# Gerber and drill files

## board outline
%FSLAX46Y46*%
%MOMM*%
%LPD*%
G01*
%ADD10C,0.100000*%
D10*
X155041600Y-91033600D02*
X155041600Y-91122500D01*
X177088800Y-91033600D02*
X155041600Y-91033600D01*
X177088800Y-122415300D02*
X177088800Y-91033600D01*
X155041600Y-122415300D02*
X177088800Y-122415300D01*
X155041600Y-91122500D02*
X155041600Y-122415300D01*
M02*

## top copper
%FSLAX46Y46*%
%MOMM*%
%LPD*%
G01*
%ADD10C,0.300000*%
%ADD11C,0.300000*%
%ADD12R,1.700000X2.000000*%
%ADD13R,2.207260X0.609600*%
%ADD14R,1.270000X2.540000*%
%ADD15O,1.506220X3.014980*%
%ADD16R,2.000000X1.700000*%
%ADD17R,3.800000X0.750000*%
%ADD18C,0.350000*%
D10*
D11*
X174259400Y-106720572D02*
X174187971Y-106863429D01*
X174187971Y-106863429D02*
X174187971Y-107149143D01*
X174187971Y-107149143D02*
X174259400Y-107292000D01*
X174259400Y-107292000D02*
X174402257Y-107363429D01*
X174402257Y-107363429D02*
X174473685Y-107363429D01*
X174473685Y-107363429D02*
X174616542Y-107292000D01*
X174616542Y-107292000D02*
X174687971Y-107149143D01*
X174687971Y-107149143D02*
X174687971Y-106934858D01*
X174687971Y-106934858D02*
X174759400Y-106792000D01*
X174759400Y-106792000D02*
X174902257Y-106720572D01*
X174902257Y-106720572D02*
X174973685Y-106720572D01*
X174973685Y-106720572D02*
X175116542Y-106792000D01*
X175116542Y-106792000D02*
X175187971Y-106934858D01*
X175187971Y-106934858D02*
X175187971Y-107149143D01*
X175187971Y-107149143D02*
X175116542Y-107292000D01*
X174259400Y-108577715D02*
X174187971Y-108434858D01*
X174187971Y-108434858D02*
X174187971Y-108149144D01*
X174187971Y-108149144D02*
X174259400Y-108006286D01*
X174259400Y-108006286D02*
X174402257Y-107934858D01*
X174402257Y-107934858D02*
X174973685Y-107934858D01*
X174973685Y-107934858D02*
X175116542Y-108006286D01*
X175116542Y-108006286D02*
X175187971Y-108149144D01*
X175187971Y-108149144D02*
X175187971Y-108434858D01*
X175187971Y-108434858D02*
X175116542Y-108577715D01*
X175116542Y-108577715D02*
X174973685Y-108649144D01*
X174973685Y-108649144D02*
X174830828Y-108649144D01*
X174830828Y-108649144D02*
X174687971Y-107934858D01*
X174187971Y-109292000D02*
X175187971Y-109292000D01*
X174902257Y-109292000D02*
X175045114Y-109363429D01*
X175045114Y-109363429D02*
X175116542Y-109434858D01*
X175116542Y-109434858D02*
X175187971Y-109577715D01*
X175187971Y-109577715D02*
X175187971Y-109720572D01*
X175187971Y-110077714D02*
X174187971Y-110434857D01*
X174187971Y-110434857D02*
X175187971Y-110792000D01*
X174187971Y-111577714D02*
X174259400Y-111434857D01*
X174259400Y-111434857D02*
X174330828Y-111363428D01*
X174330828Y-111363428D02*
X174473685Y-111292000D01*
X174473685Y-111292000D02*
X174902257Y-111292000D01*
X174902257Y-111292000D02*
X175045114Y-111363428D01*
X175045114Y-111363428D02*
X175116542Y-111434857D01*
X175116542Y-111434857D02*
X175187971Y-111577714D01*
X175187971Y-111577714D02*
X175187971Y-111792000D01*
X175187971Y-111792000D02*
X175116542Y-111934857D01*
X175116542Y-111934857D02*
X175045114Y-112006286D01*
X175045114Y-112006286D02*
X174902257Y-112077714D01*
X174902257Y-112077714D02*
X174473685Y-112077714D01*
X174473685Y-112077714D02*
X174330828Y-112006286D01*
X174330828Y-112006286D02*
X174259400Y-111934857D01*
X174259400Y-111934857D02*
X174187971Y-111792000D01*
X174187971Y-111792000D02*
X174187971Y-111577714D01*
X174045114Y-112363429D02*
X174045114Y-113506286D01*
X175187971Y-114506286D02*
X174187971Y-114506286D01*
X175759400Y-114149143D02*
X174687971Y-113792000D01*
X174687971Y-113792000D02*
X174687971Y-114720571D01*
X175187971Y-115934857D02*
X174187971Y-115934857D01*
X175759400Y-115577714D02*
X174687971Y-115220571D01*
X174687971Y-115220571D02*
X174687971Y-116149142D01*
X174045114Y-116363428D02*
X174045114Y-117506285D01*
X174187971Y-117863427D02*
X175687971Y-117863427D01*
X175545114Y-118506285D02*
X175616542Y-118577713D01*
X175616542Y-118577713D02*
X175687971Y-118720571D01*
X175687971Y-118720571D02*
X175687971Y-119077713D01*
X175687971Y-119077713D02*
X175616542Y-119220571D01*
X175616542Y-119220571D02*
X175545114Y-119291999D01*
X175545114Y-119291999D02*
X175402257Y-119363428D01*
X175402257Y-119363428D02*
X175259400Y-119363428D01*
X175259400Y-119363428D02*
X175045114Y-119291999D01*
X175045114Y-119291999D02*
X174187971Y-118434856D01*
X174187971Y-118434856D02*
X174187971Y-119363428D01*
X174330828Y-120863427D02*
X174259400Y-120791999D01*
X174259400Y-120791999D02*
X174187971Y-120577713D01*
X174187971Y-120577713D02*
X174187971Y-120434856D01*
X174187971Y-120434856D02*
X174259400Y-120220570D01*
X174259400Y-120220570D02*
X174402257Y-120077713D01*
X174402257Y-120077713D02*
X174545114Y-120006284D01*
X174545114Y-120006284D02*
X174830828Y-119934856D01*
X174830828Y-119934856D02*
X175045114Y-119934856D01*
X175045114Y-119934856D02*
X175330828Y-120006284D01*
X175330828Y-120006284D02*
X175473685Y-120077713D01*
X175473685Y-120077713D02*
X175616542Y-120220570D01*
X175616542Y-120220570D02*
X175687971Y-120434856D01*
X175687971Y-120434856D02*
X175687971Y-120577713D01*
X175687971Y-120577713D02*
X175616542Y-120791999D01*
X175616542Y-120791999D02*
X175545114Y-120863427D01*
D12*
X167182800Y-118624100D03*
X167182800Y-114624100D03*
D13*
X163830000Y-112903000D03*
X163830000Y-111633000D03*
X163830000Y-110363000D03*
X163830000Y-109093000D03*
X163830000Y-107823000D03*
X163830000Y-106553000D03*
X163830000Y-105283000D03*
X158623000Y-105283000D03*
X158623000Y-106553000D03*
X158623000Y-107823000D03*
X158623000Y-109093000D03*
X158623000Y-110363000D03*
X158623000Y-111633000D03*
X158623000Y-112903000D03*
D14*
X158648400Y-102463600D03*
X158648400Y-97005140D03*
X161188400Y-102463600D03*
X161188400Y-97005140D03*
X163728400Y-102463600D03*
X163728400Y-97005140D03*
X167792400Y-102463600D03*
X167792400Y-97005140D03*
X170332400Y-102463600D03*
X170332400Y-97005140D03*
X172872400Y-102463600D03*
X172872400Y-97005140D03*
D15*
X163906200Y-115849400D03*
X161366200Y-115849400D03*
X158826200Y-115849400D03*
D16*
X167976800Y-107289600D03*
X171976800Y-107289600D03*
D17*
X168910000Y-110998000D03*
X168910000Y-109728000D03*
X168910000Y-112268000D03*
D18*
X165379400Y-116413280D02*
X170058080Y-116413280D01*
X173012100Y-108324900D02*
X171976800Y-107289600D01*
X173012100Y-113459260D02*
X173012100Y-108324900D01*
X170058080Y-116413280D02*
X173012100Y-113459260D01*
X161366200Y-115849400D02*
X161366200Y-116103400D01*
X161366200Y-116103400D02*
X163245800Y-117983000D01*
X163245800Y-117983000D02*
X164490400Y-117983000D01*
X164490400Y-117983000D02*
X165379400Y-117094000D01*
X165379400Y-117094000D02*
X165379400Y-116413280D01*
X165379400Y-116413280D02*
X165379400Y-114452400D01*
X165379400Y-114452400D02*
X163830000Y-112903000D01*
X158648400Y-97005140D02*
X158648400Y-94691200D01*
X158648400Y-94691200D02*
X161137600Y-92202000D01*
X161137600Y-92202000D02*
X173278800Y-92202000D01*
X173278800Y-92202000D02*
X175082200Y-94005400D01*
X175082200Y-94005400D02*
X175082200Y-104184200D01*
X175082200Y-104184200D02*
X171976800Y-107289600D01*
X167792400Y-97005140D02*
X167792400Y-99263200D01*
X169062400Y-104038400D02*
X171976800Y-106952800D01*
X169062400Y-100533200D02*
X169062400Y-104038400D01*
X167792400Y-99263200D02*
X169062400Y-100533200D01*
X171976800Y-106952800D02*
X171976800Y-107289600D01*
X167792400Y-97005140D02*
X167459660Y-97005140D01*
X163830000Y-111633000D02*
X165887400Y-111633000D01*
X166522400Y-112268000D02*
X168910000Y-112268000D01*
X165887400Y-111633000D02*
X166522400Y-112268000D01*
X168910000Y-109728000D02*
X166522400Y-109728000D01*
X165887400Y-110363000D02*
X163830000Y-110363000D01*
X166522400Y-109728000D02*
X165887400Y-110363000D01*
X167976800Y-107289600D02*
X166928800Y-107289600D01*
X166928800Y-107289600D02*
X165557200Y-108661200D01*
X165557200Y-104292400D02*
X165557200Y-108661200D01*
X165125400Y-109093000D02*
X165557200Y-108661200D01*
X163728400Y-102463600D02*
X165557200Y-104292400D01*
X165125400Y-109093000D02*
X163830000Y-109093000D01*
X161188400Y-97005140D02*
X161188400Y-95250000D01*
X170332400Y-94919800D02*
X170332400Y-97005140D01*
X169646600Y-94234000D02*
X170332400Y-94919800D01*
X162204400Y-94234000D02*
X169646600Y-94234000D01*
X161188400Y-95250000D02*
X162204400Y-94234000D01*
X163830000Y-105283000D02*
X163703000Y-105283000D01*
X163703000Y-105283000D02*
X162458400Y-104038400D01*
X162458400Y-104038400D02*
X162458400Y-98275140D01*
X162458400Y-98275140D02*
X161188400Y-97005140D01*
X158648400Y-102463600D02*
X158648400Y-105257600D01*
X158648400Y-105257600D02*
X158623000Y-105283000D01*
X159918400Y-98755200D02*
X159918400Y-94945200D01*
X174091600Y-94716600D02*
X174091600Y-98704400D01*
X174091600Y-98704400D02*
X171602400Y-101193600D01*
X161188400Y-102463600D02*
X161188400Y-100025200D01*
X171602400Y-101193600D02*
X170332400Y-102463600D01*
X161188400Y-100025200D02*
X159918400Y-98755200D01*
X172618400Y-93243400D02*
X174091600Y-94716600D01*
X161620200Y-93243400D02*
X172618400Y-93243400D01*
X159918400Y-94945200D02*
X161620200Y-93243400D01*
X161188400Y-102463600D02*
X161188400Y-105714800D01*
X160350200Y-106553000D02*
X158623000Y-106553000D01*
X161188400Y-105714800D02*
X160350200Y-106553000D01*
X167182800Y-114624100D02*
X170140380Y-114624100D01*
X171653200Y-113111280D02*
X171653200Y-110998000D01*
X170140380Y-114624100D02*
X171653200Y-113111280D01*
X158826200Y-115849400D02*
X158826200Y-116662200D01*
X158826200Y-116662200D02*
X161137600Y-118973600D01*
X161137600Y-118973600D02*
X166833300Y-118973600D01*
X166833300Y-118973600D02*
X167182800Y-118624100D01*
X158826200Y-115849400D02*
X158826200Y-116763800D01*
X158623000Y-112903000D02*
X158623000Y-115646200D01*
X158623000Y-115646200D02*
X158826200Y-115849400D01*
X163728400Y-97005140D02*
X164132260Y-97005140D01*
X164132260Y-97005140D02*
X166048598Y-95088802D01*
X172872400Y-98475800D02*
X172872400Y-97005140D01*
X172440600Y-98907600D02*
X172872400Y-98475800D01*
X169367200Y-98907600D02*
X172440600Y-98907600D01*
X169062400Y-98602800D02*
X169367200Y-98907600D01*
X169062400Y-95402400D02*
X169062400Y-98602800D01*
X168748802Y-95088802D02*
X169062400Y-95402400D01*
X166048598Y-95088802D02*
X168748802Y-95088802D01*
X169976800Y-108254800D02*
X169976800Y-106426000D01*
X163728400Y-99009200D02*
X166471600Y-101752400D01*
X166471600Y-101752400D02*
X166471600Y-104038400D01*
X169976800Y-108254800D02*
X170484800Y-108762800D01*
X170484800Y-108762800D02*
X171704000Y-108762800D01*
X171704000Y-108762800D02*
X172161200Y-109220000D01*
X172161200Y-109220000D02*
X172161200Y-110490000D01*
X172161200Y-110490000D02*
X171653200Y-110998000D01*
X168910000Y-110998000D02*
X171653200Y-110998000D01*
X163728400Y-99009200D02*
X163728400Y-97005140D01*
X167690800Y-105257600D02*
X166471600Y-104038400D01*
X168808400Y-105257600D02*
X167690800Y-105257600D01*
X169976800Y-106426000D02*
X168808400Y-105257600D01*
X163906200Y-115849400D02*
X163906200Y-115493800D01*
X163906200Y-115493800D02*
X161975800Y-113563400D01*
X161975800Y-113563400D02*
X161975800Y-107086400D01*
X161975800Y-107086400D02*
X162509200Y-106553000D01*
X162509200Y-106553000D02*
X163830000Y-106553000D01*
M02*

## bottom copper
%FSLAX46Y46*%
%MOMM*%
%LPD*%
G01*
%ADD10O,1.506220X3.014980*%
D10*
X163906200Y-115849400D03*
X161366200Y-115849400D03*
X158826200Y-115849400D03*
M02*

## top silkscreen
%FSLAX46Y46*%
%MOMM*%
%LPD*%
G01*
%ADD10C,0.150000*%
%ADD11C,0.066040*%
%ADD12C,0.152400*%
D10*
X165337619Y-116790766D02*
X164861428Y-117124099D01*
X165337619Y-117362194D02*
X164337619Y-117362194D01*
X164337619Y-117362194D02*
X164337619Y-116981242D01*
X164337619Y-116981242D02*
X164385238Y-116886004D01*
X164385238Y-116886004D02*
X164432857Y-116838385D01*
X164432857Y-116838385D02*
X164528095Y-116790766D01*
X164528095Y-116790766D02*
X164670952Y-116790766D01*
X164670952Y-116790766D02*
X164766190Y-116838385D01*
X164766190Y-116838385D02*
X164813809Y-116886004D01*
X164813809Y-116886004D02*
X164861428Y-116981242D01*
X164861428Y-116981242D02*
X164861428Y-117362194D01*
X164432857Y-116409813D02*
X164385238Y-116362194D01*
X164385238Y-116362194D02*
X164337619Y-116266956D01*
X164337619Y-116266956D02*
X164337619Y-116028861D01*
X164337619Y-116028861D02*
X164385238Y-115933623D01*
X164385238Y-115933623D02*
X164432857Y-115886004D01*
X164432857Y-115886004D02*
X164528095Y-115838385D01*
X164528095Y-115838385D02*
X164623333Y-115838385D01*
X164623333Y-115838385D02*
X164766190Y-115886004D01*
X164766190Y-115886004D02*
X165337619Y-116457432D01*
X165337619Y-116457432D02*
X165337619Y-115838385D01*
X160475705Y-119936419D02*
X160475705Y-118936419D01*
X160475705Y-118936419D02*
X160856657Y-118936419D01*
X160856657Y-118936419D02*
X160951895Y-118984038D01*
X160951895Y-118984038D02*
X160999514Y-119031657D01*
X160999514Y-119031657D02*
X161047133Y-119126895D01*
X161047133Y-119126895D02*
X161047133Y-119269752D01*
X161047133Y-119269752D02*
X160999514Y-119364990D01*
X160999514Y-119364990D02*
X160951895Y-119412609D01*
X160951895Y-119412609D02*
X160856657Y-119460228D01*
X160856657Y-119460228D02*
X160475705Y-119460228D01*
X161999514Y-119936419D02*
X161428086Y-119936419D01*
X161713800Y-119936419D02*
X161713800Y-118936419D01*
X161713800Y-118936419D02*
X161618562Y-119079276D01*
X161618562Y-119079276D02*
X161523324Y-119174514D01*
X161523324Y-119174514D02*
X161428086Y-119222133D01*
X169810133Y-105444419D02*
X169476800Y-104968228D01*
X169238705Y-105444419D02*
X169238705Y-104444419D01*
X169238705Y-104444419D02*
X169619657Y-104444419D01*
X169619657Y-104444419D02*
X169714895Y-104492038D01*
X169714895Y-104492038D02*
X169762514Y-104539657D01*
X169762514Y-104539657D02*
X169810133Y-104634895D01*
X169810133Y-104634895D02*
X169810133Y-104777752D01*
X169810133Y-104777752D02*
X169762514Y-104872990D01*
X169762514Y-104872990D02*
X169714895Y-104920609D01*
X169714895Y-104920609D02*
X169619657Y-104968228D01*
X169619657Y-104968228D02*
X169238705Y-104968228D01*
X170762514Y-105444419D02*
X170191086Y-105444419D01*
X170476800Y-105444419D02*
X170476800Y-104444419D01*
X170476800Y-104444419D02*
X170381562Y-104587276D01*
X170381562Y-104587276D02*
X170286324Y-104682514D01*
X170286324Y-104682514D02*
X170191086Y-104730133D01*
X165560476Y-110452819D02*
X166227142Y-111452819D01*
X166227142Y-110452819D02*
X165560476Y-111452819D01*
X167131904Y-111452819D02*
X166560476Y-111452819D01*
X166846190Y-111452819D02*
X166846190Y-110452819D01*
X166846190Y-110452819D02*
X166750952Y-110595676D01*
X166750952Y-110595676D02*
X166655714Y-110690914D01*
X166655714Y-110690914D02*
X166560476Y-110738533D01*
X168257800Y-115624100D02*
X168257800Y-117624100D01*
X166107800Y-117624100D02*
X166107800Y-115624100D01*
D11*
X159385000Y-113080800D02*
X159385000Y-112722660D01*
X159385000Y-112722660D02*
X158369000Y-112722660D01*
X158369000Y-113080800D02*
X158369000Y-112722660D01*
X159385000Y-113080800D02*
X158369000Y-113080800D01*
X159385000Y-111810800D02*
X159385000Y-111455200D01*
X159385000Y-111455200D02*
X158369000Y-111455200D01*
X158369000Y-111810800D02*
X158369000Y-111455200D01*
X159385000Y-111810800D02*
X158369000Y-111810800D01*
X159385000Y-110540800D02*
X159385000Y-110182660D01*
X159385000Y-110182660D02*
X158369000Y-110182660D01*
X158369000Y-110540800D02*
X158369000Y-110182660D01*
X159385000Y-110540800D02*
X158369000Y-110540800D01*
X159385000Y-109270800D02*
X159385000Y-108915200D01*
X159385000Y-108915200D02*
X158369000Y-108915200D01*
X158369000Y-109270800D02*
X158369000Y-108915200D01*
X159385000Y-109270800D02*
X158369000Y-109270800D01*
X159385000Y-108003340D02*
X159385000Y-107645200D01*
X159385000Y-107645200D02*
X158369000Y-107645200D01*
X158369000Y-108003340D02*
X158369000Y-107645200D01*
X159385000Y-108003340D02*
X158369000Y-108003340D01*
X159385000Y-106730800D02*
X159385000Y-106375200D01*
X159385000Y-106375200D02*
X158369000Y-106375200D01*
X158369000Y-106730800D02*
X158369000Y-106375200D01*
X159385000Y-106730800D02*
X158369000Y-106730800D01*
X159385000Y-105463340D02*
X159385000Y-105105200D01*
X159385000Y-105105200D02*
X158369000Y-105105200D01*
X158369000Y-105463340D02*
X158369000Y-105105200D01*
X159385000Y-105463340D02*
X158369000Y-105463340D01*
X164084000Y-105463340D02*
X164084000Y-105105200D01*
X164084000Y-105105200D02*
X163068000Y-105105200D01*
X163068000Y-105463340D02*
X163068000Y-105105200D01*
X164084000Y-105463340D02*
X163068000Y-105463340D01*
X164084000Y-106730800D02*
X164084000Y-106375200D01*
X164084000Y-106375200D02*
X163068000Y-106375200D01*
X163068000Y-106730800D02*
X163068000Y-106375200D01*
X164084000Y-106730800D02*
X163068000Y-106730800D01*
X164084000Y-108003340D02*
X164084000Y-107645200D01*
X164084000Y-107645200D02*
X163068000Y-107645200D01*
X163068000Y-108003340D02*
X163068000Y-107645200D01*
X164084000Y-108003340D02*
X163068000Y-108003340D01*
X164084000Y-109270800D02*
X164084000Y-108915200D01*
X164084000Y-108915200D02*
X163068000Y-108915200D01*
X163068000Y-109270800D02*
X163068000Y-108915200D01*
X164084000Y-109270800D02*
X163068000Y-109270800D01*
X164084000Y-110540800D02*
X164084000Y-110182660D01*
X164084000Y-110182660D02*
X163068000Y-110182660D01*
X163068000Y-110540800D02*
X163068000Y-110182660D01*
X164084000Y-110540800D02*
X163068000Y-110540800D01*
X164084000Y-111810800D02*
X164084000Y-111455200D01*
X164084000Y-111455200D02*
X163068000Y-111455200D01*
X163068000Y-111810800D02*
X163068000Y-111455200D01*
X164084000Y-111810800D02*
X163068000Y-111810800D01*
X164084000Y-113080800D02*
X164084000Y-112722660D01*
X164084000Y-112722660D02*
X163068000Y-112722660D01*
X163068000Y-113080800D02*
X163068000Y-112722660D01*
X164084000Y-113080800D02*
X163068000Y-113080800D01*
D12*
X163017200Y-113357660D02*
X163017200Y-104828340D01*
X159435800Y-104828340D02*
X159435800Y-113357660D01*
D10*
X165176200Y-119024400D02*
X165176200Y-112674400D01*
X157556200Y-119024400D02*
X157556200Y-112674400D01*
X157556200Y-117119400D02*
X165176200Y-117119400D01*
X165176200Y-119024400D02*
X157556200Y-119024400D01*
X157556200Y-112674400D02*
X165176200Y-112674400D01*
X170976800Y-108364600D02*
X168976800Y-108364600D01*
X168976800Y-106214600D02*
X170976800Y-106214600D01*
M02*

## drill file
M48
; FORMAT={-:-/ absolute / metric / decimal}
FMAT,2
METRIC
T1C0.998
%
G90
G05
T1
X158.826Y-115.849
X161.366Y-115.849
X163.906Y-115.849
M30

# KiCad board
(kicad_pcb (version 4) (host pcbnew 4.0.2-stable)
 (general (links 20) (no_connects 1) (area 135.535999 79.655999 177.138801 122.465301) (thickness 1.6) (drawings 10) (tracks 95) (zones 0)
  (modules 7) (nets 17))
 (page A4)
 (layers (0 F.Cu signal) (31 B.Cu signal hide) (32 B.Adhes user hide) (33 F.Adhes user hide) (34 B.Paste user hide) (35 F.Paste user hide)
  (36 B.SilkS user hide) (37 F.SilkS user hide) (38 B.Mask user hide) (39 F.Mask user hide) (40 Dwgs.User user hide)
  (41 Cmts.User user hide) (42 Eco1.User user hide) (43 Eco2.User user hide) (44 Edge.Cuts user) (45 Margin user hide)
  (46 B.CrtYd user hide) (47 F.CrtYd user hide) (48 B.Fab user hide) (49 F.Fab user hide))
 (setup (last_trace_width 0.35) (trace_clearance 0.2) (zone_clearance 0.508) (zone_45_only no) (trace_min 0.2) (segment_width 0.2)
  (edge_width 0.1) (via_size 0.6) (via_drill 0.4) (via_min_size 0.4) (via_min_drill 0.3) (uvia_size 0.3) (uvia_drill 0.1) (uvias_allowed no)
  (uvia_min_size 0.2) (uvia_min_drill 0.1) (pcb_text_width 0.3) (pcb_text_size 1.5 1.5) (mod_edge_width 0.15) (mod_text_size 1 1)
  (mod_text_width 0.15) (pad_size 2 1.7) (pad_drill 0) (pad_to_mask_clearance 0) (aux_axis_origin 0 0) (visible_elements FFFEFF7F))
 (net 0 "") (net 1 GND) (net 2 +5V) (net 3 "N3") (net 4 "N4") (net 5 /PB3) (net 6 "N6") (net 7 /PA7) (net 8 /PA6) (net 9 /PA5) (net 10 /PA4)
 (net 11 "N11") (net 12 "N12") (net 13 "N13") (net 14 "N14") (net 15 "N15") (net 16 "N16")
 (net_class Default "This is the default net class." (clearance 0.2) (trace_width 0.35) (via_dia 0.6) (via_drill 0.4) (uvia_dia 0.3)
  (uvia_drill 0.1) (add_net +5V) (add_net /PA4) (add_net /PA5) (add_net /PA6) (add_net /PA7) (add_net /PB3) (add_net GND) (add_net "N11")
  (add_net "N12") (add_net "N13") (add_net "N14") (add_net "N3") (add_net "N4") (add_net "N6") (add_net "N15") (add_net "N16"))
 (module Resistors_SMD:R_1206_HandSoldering (layer F.Cu) (at 167.1828 116.6241 90)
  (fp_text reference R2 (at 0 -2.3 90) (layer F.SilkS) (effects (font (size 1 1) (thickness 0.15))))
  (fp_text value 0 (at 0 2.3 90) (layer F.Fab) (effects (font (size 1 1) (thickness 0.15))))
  (fp_line (start 1 1.075) (end -1 1.075) (layer F.SilkS) (width 0.15))
  (fp_line (start -1 -1.075) (end 1 -1.075) (layer F.SilkS) (width 0.15))
  (pad 2 smd rect (at -2 0 90) (size 2 1.7) (layers F.Cu F.Paste F.Mask) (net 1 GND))
  (pad 1 smd rect (at 2 0 90) (size 2 1.7) (layers F.Cu F.Paste F.Mask) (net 1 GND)))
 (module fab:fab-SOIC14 (layer F.Cu) (at 161.2265 109.093 90)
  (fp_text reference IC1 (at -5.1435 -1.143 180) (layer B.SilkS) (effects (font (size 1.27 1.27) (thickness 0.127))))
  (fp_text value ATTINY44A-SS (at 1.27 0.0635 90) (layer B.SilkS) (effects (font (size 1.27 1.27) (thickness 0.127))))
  (fp_line (start -3.9878 -1.8415) (end -3.62966 -1.8415) (layer F.SilkS) (width 0.06604))
  (fp_line (start -3.62966 -1.8415) (end -3.62966 -2.8575) (layer F.SilkS) (width 0.06604))
  (fp_line (start -3.9878 -2.8575) (end -3.62966 -2.8575) (layer F.SilkS) (width 0.06604))
  (fp_line (start -3.9878 -1.8415) (end -3.9878 -2.8575) (layer F.SilkS) (width 0.06604))
  (fp_line (start -2.7178 -1.8415) (end -2.3622 -1.8415) (layer F.SilkS) (width 0.06604))
  (fp_line (start -2.3622 -1.8415) (end -2.3622 -2.8575) (layer F.SilkS) (width 0.06604))
  (fp_line (start -2.7178 -2.8575) (end -2.3622 -2.8575) (layer F.SilkS) (width 0.06604))
  (fp_line (start -2.7178 -1.8415) (end -2.7178 -2.8575) (layer F.SilkS) (width 0.06604))
  (fp_line (start -1.4478 -1.8415) (end -1.08966 -1.8415) (layer F.SilkS) (width 0.06604))
  (fp_line (start -1.08966 -1.8415) (end -1.08966 -2.8575) (layer F.SilkS) (width 0.06604))
  (fp_line (start -1.4478 -2.8575) (end -1.08966 -2.8575) (layer F.SilkS) (width 0.06604))
  (fp_line (start -1.4478 -1.8415) (end -1.4478 -2.8575) (layer F.SilkS) (width 0.06604))
  (fp_line (start -0.1778 -1.8415) (end 0.1778 -1.8415) (layer F.SilkS) (width 0.06604))
  (fp_line (start 0.1778 -1.8415) (end 0.1778 -2.8575) (layer F.SilkS) (width 0.06604))
  (fp_line (start -0.1778 -2.8575) (end 0.1778 -2.8575) (layer F.SilkS) (width 0.06604))
  (fp_line (start -0.1778 -1.8415) (end -0.1778 -2.8575) (layer F.SilkS) (width 0.06604))
  (fp_line (start 1.08966 -1.8415) (end 1.4478 -1.8415) (layer F.SilkS) (width 0.06604))
  (fp_line (start 1.4478 -1.8415) (end 1.4478 -2.8575) (layer F.SilkS) (width 0.06604))
  (fp_line (start 1.08966 -2.8575) (end 1.4478 -2.8575) (layer F.SilkS) (width 0.06604))
  (fp_line (start 1.08966 -1.8415) (end 1.08966 -2.8575) (layer F.SilkS) (width 0.06604))
  (fp_line (start 2.3622 -1.8415) (end 2.7178 -1.8415) (layer F.SilkS) (width 0.06604))
  (fp_line (start 2.7178 -1.8415) (end 2.7178 -2.8575) (layer F.SilkS) (width 0.06604))
  (fp_line (start 2.3622 -2.8575) (end 2.7178 -2.8575) (layer F.SilkS) (width 0.06604))
  (fp_line (start 2.3622 -1.8415) (end 2.3622 -2.8575) (layer F.SilkS) (width 0.06604))
  (fp_line (start 3.62966 -1.8415) (end 3.9878 -1.8415) (layer F.SilkS) (width 0.06604))
  (fp_line (start 3.9878 -1.8415) (end 3.9878 -2.8575) (layer F.SilkS) (width 0.06604))
  (fp_line (start 3.62966 -2.8575) (end 3.9878 -2.8575) (layer F.SilkS) (width 0.06604))
  (fp_line (start 3.62966 -1.8415) (end 3.62966 -2.8575) (layer F.SilkS) (width 0.06604))
  (fp_line (start 3.62966 2.8575) (end 3.9878 2.8575) (layer F.SilkS) (width 0.06604))
  (fp_line (start 3.9878 2.8575) (end 3.9878 1.8415) (layer F.SilkS) (width 0.06604))
  (fp_line (start 3.62966 1.8415) (end 3.9878 1.8415) (layer F.SilkS) (width 0.06604))
  (fp_line (start 3.62966 2.8575) (end 3.62966 1.8415) (layer F.SilkS) (width 0.06604))
  (fp_line (start 2.3622 2.8575) (end 2.7178 2.8575) (layer F.SilkS) (width 0.06604))
  (fp_line (start 2.7178 2.8575) (end 2.7178 1.8415) (layer F.SilkS) (width 0.06604))
  (fp_line (start 2.3622 1.8415) (end 2.7178 1.8415) (layer F.SilkS) (width 0.06604))
  (fp_line (start 2.3622 2.8575) (end 2.3622 1.8415) (layer F.SilkS) (width 0.06604))
  (fp_line (start 1.08966 2.8575) (end 1.4478 2.8575) (layer F.SilkS) (width 0.06604))
  (fp_line (start 1.4478 2.8575) (end 1.4478 1.8415) (layer F.SilkS) (width 0.06604))
  (fp_line (start 1.08966 1.8415) (end 1.4478 1.8415) (layer F.SilkS) (width 0.06604))
  (fp_line (start 1.08966 2.8575) (end 1.08966 1.8415) (layer F.SilkS) (width 0.06604))
  (fp_line (start -0.1778 2.8575) (end 0.1778 2.8575) (layer F.SilkS) (width 0.06604))
  (fp_line (start 0.1778 2.8575) (end 0.1778 1.8415) (layer F.SilkS) (width 0.06604))
  (fp_line (start -0.1778 1.8415) (end 0.1778 1.8415) (layer F.SilkS) (width 0.06604))
  (fp_line (start -0.1778 2.8575) (end -0.1778 1.8415) (layer F.SilkS) (width 0.06604))
  (fp_line (start -1.4478 2.8575) (end -1.08966 2.8575) (layer F.SilkS) (width 0.06604))
  (fp_line (start -1.08966 2.8575) (end -1.08966 1.8415) (layer F.SilkS) (width 0.06604))
  (fp_line (start -1.4478 1.8415) (end -1.08966 1.8415) (layer F.SilkS) (width 0.06604))
  (fp_line (start -1.4478 2.8575) (end -1.4478 1.8415) (layer F.SilkS) (width 0.06604))
  (fp_line (start -2.7178 2.8575) (end -2.3622 2.8575) (layer F.SilkS) (width 0.06604))
  (fp_line (start -2.3622 2.8575) (end -2.3622 1.8415) (layer F.SilkS) (width 0.06604))
  (fp_line (start -2.7178 1.8415) (end -2.3622 1.8415) (layer F.SilkS) (width 0.06604))
  (fp_line (start -2.7178 2.8575) (end -2.7178 1.8415) (layer F.SilkS) (width 0.06604))
  (fp_line (start -3.9878 2.8575) (end -3.62966 2.8575) (layer F.SilkS) (width 0.06604))
  (fp_line (start -3.62966 2.8575) (end -3.62966 1.8415) (layer F.SilkS) (width 0.06604))
  (fp_line (start -3.9878 1.8415) (end -3.62966 1.8415) (layer F.SilkS) (width 0.06604))
  (fp_line (start -3.9878 2.8575) (end -3.9878 1.8415) (layer F.SilkS) (width 0.06604))
  (fp_line (start -4.26466 1.7907) (end 4.26466 1.7907) (layer F.SilkS) (width 0.1524))
  (fp_line (start 4.26466 -1.7907) (end -4.26466 -1.7907) (layer F.SilkS) (width 0.1524))
  (pad 1 smd rect (at -3.81 2.6035 90) (size 0.6096 2.20726) (layers F.Cu F.Paste F.Mask) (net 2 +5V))
  (pad 2 smd rect (at -2.54 2.6035 90) (size 0.6096 2.20726) (layers F.Cu F.Paste F.Mask) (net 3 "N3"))
  (pad 3 smd rect (at -1.27 2.6035 90) (size 0.6096 2.20726) (layers F.Cu F.Paste F.Mask) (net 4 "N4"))
  (pad 4 smd rect (at 0 2.6035 90) (size 0.6096 2.20726) (layers F.Cu F.Paste F.Mask) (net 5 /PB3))
  (pad 5 smd rect (at 1.27 2.6035 90) (size 0.6096 2.20726) (layers F.Cu F.Paste F.Mask) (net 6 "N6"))
  (pad 6 smd rect (at 2.54 2.6035 90) (size 0.6096 2.20726) (layers F.Cu F.Paste F.Mask) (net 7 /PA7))
  (pad 7 smd rect (at 3.81 2.6035 90) (size 0.6096 2.20726) (layers F.Cu F.Paste F.Mask) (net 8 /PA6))
  (pad 8 smd rect (at 3.81 -2.6035 90) (size 0.6096 2.20726) (layers F.Cu F.Paste F.Mask) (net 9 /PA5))
  (pad 9 smd rect (at 2.54 -2.6035 90) (size 0.6096 2.20726) (layers F.Cu F.Paste F.Mask) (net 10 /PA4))
  (pad 10 smd rect (at 1.27 -2.6035 90) (size 0.6096 2.20726) (layers F.Cu F.Paste F.Mask) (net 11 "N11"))
  (pad 11 smd rect (at 0 -2.6035 90) (size 0.6096 2.20726) (layers F.Cu F.Paste F.Mask) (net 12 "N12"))
  (pad 12 smd rect (at -1.27 -2.6035 90) (size 0.6096 2.20726) (layers F.Cu F.Paste F.Mask) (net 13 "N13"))
  (pad 13 smd rect (at -2.54 -2.6035 90) (size 0.6096 2.20726) (layers F.Cu F.Paste F.Mask) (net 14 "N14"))
  (pad 14 smd rect (at -3.81 -2.6035 90) (size 0.6096 2.20726) (layers F.Cu F.Paste F.Mask) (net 1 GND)))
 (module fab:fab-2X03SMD (layer F.Cu) (at 161.1884 99.9236 90)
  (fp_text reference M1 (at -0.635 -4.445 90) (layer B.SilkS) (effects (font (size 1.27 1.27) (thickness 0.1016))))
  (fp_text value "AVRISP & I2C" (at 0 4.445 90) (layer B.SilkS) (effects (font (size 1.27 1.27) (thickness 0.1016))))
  (pad 1 smd rect (at -2.54 -2.54 90) (size 2.54 1.27) (layers F.Cu F.Paste F.Mask) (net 9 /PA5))
  (pad 2 smd rect (at 2.91846 -2.54 90) (size 2.54 1.27) (layers F.Cu F.Paste F.Mask) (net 2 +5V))
  (pad 3 smd rect (at -2.54 0 90) (size 2.54 1.27) (layers F.Cu F.Paste F.Mask) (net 10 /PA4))
  (pad 4 smd rect (at 2.91846 0 90) (size 2.54 1.27) (layers F.Cu F.Paste F.Mask) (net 8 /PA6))
  (pad 5 smd rect (at -2.54 2.54 90) (size 2.54 1.27) (layers F.Cu F.Paste F.Mask) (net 5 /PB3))
  (pad 6 smd rect (at 2.91846 2.54 90) (size 2.54 1.27) (layers F.Cu F.Paste F.Mask) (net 1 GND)))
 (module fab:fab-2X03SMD (layer F.Cu) (at 170.3324 99.9236 90)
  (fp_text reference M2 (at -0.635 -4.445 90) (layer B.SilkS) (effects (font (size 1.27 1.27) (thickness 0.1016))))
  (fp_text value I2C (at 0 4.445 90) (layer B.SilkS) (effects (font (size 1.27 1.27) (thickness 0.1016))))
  (pad 1 smd rect (at -2.54 -2.54 90) (size 2.54 1.27) (layers F.Cu F.Paste F.Mask) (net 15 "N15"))
  (pad 2 smd rect (at 2.91846 -2.54 90) (size 2.54 1.27) (layers F.Cu F.Paste F.Mask) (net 2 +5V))
  (pad 3 smd rect (at -2.54 0 90) (size 2.54 1.27) (layers F.Cu F.Paste F.Mask) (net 10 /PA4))
  (pad 4 smd rect (at 2.91846 0 90) (size 2.54 1.27) (layers F.Cu F.Paste F.Mask) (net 8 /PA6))
  (pad 5 smd rect (at -2.54 2.54 90) (size 2.54 1.27) (layers F.Cu F.Paste F.Mask) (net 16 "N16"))
  (pad 6 smd rect (at 2.91846 2.54 90) (size 2.54 1.27) (layers F.Cu F.Paste F.Mask) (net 1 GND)))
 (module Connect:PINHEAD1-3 (layer F.Cu) (at 161.3662 115.8494 180)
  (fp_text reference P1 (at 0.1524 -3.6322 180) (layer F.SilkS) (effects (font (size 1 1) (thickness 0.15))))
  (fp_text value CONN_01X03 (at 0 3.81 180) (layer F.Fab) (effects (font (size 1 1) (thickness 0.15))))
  (fp_line (start -3.81 -3.175) (end -3.81 3.175) (layer F.SilkS) (width 0.15))
  (fp_line (start 3.81 -3.175) (end 3.81 3.175) (layer F.SilkS) (width 0.15))
  (fp_line (start 3.81 -1.27) (end -3.81 -1.27) (layer F.SilkS) (width 0.15))
  (fp_line (start -3.81 -3.175) (end 3.81 -3.175) (layer F.SilkS) (width 0.15))
  (fp_line (start 3.81 3.175) (end -3.81 3.175) (layer F.SilkS) (width 0.15))
  (pad 1 thru_hole oval (at -2.54 0 180) (size 1.50622 3.01498) (drill 0.99822) (layers *.Cu *.Mask) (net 7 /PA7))
  (pad 2 thru_hole oval (at 0 0 180) (size 1.50622 3.01498) (drill 0.99822) (layers *.Cu *.Mask) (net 2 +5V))
  (pad 3 thru_hole oval (at 2.54 0 180) (size 1.50622 3.01498) (drill 0.99822) (layers *.Cu *.Mask) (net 1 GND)))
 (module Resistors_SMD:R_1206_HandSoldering (layer F.Cu) (at 169.9768 107.2896)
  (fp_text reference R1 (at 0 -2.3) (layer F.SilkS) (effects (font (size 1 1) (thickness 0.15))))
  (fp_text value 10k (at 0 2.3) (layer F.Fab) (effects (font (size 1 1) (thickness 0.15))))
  (fp_line (start 1 1.075) (end -1 1.075) (layer F.SilkS) (width 0.15))
  (fp_line (start -1 -1.075) (end 1 -1.075) (layer F.SilkS) (width 0.15))
  (pad 1 smd rect (at -2 0) (size 2 1.7) (layers F.Cu F.Paste F.Mask) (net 5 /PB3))
  (pad 2 smd rect (at 2 0) (size 2 1.7) (layers F.Cu F.Paste F.Mask) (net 2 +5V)))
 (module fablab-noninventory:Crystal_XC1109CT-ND (layer F.Cu) (at 168.91 110.998 90)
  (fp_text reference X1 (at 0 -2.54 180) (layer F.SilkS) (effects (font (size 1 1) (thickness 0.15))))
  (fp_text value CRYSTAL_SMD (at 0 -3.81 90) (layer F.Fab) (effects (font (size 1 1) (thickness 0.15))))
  (pad 2 smd rect (at 0 0 90) (size 0.75 3.8) (layers F.Cu F.Paste F.Mask) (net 1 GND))
  (pad 1 smd rect (at 1.27 0 90) (size 0.75 3.8) (layers F.Cu F.Paste F.Mask) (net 4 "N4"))
  (pad 3 smd rect (at -1.27 0 90) (size 0.75 3.8) (layers F.Cu F.Paste F.Mask) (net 3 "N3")))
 (gr_line (start 155.0416 91.0336) (end 155.0416 91.1225) (angle 90) (layer Edge.Cuts) (width 0.1))
 (gr_line (start 177.0888 91.0336) (end 155.0416 91.0336) (angle 90) (layer Edge.Cuts) (width 0.1))
 (gr_line (start 177.0888 122.4153) (end 177.0888 91.0336) (angle 90) (layer Edge.Cuts) (width 0.1))
 (gr_line (start 155.0416 122.4153) (end 177.0888 122.4153) (angle 90) (layer Edge.Cuts) (width 0.1))
 (gr_line (start 155.0416 91.1225) (end 155.0416 122.4153) (angle 90) (layer Edge.Cuts) (width 0.1))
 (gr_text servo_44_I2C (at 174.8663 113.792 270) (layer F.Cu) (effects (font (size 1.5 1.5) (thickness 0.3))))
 (segment (start 165.3794 116.41328) (end 170.05808 116.41328) (width 0.35) (layer F.Cu) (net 2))
 (segment (start 173.0121 108.3249) (end 171.9768 107.2896) (width 0.35) (layer F.Cu) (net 2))
 (segment (start 173.0121 113.45926) (end 173.0121 108.3249) (width 0.35) (layer F.Cu) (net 2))
 (segment (start 170.05808 116.41328) (end 173.0121 113.45926) (width 0.35) (layer F.Cu) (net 2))
 (segment (start 161.3662 115.8494) (end 161.3662 116.1034) (width 0.35) (layer F.Cu) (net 2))
 (segment (start 161.3662 116.1034) (end 163.2458 117.983) (width 0.35) (layer F.Cu) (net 2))
 (segment (start 163.2458 117.983) (end 164.4904 117.983) (width 0.35) (layer F.Cu) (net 2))
 (segment (start 164.4904 117.983) (end 165.3794 117.094) (width 0.35) (layer F.Cu) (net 2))
 (segment (start 165.3794 117.094) (end 165.3794 116.41328) (width 0.35) (layer F.Cu) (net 2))
 (segment (start 165.3794 116.41328) (end 165.3794 114.4524) (width 0.35) (layer F.Cu) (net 2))
 (segment (start 165.3794 114.4524) (end 163.83 112.903) (width 0.35) (layer F.Cu) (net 2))
 (segment (start 158.6484 97.00514) (end 158.6484 94.6912) (width 0.35) (layer F.Cu) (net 2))
 (segment (start 158.6484 94.6912) (end 161.1376 92.202) (width 0.35) (layer F.Cu) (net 2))
 (segment (start 161.1376 92.202) (end 173.2788 92.202) (width 0.35) (layer F.Cu) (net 2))
 (segment (start 173.2788 92.202) (end 175.0822 94.0054) (width 0.35) (layer F.Cu) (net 2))
 (segment (start 175.0822 94.0054) (end 175.0822 104.1842) (width 0.35) (layer F.Cu) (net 2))
 (segment (start 175.0822 104.1842) (end 171.9768 107.2896) (width 0.35) (layer F.Cu) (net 2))
 (segment (start 167.7924 97.00514) (end 167.7924 99.2632) (width 0.35) (layer F.Cu) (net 2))
 (segment (start 169.0624 104.0384) (end 171.9768 106.9528) (width 0.35) (layer F.Cu) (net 2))
 (segment (start 169.0624 100.5332) (end 169.0624 104.0384) (width 0.35) (layer F.Cu) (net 2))
 (segment (start 167.7924 99.2632) (end 169.0624 100.5332) (width 0.35) (layer F.Cu) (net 2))
 (segment (start 171.9768 106.9528) (end 171.9768 107.2896) (width 0.35) (layer F.Cu) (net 2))
 (segment (start 167.7924 97.00514) (end 167.45966 97.00514) (width 0.35) (layer F.Cu) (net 2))
 (segment (start 163.83 111.633) (end 165.8874 111.633) (width 0.35) (layer F.Cu) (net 3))
 (segment (start 166.5224 112.268) (end 168.91 112.268) (width 0.35) (layer F.Cu) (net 3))
 (segment (start 165.8874 111.633) (end 166.5224 112.268) (width 0.35) (layer F.Cu) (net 3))
 (segment (start 168.91 109.728) (end 166.5224 109.728) (width 0.35) (layer F.Cu) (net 4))
 (segment (start 165.8874 110.363) (end 163.83 110.363) (width 0.35) (layer F.Cu) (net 4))
 (segment (start 166.5224 109.728) (end 165.8874 110.363) (width 0.35) (layer F.Cu) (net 4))
 (segment (start 167.9768 107.2896) (end 166.9288 107.2896) (width 0.35) (layer F.Cu) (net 5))
 (segment (start 166.9288 107.2896) (end 165.5572 108.6612) (width 0.35) (layer F.Cu) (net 5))
 (segment (start 165.5572 104.2924) (end 165.5572 108.6612) (width 0.35) (layer F.Cu) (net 5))
 (segment (start 165.1254 109.093) (end 165.5572 108.6612) (width 0.35) (layer F.Cu) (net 5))
 (segment (start 163.7284 102.4636) (end 165.5572 104.2924) (width 0.35) (layer F.Cu) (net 5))
 (segment (start 165.1254 109.093) (end 163.83 109.093) (width 0.35) (layer F.Cu) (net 5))
 (segment (start 161.1884 97.00514) (end 161.1884 95.25) (width 0.35) (layer F.Cu) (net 8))
 (segment (start 170.3324 94.9198) (end 170.3324 97.00514) (width 0.35) (layer F.Cu) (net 8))
 (segment (start 169.6466 94.234) (end 170.3324 94.9198) (width 0.35) (layer F.Cu) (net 8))
 (segment (start 162.2044 94.234) (end 169.6466 94.234) (width 0.35) (layer F.Cu) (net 8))
 (segment (start 161.1884 95.25) (end 162.2044 94.234) (width 0.35) (layer F.Cu) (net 8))
 (segment (start 163.83 105.283) (end 163.703 105.283) (width 0.35) (layer F.Cu) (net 8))
 (segment (start 163.703 105.283) (end 162.4584 104.0384) (width 0.35) (layer F.Cu) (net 8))
 (segment (start 162.4584 104.0384) (end 162.4584 98.27514) (width 0.35) (layer F.Cu) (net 8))
 (segment (start 162.4584 98.27514) (end 161.1884 97.00514) (width 0.35) (layer F.Cu) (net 8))
 (segment (start 158.6484 102.4636) (end 158.6484 105.2576) (width 0.35) (layer F.Cu) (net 9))
 (segment (start 158.6484 105.2576) (end 158.623 105.283) (width 0.35) (layer F.Cu) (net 9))
 (segment (start 159.9184 98.7552) (end 159.9184 94.9452) (width 0.35) (layer F.Cu) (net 10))
 (segment (start 174.0916 94.7166) (end 174.0916 98.7044) (width 0.35) (layer F.Cu) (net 10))
 (segment (start 174.0916 98.7044) (end 171.6024 101.1936) (width 0.35) (layer F.Cu) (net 10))
 (segment (start 161.1884 102.4636) (end 161.1884 100.0252) (width 0.35) (layer F.Cu) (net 10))
 (segment (start 171.6024 101.1936) (end 170.3324 102.4636) (width 0.35) (layer F.Cu) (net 10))
 (segment (start 161.1884 100.0252) (end 159.9184 98.7552) (width 0.35) (layer F.Cu) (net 10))
 (segment (start 172.6184 93.2434) (end 174.0916 94.7166) (width 0.35) (layer F.Cu) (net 10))
 (segment (start 161.6202 93.2434) (end 172.6184 93.2434) (width 0.35) (layer F.Cu) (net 10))
 (segment (start 159.9184 94.9452) (end 161.6202 93.2434) (width 0.35) (layer F.Cu) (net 10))
 (segment (start 161.1884 102.4636) (end 161.1884 105.7148) (width 0.35) (layer F.Cu) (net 10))
 (segment (start 160.3502 106.553) (end 158.623 106.553) (width 0.35) (layer F.Cu) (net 10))
 (segment (start 161.1884 105.7148) (end 160.3502 106.553) (width 0.35) (layer F.Cu) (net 10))
 (segment (start 167.1828 114.6241) (end 170.14038 114.6241) (width 0.35) (layer F.Cu) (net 1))
 (segment (start 171.6532 113.11128) (end 171.6532 110.998) (width 0.35) (layer F.Cu) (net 1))
 (segment (start 170.14038 114.6241) (end 171.6532 113.11128) (width 0.35) (layer F.Cu) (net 1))
 (segment (start 158.8262 115.8494) (end 158.8262 116.6622) (width 0.35) (layer F.Cu) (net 1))
 (segment (start 158.8262 116.6622) (end 161.1376 118.9736) (width 0.35) (layer F.Cu) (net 1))
 (segment (start 161.1376 118.9736) (end 166.8333 118.9736) (width 0.35) (layer F.Cu) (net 1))
 (segment (start 166.8333 118.9736) (end 167.1828 118.6241) (width 0.35) (layer F.Cu) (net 1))
 (segment (start 158.8262 115.8494) (end 158.8262 116.7638) (width 0.35) (layer F.Cu) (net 1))
 (segment (start 158.623 112.903) (end 158.623 115.6462) (width 0.35) (layer F.Cu) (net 1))
 (segment (start 158.623 115.6462) (end 158.8262 115.8494) (width 0.35) (layer F.Cu) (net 1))
 (segment (start 163.7284 97.00514) (end 164.13226 97.00514) (width 0.35) (layer F.Cu) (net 1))
 (segment (start 164.13226 97.00514) (end 166.048598 95.088802) (width 0.35) (layer F.Cu) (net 1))
 (segment (start 172.8724 98.4758) (end 172.8724 97.00514) (width 0.35) (layer F.Cu) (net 1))
 (segment (start 172.4406 98.9076) (end 172.8724 98.4758) (width 0.35) (layer F.Cu) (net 1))
 (segment (start 169.3672 98.9076) (end 172.4406 98.9076) (width 0.35) (layer F.Cu) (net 1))
 (segment (start 169.0624 98.6028) (end 169.3672 98.9076) (width 0.35) (layer F.Cu) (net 1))
 (segment (start 169.0624 95.4024) (end 169.0624 98.6028) (width 0.35) (layer F.Cu) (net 1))
 (segment (start 168.748802 95.088802) (end 169.0624 95.4024) (width 0.35) (layer F.Cu) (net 1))
 (segment (start 166.048598 95.088802) (end 168.748802 95.088802) (width 0.35) (layer F.Cu) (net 1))
 (segment (start 169.9768 108.2548) (end 169.9768 106.426) (width 0.35) (layer F.Cu) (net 1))
 (segment (start 163.7284 99.0092) (end 166.4716 101.7524) (width 0.35) (layer F.Cu) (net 1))
 (segment (start 166.4716 101.7524) (end 166.4716 104.0384) (width 0.35) (layer F.Cu) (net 1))
 (segment (start 169.9768 108.2548) (end 170.4848 108.7628) (width 0.35) (layer F.Cu) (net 1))
 (segment (start 170.4848 108.7628) (end 171.704 108.7628) (width 0.35) (layer F.Cu) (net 1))
 (segment (start 171.704 108.7628) (end 172.1612 109.22) (width 0.35) (layer F.Cu) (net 1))
 (segment (start 172.1612 109.22) (end 172.1612 110.49) (width 0.35) (layer F.Cu) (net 1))
 (segment (start 172.1612 110.49) (end 171.6532 110.998) (width 0.35) (layer F.Cu) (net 1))
 (segment (start 168.91 110.998) (end 171.6532 110.998) (width 0.35) (layer F.Cu) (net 1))
 (segment (start 163.7284 99.0092) (end 163.7284 97.00514) (width 0.35) (layer F.Cu) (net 1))
 (segment (start 167.6908 105.2576) (end 166.4716 104.0384) (width 0.35) (layer F.Cu) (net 1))
 (segment (start 168.8084 105.2576) (end 167.6908 105.2576) (width 0.35) (layer F.Cu) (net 1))
 (segment (start 169.9768 106.426) (end 168.8084 105.2576) (width 0.35) (layer F.Cu) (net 1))
 (segment (start 163.9062 115.8494) (end 163.9062 115.4938) (width 0.35) (layer F.Cu) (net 7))
 (segment (start 163.9062 115.4938) (end 161.9758 113.5634) (width 0.35) (layer F.Cu) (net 7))
 (segment (start 161.9758 113.5634) (end 161.9758 107.0864) (width 0.35) (layer F.Cu) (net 7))
 (segment (start 161.9758 107.0864) (end 162.5092 106.553) (width 0.35) (layer F.Cu) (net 7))
 (segment (start 162.5092 106.553) (end 163.83 106.553) (width 0.35) (layer F.Cu) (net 7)))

